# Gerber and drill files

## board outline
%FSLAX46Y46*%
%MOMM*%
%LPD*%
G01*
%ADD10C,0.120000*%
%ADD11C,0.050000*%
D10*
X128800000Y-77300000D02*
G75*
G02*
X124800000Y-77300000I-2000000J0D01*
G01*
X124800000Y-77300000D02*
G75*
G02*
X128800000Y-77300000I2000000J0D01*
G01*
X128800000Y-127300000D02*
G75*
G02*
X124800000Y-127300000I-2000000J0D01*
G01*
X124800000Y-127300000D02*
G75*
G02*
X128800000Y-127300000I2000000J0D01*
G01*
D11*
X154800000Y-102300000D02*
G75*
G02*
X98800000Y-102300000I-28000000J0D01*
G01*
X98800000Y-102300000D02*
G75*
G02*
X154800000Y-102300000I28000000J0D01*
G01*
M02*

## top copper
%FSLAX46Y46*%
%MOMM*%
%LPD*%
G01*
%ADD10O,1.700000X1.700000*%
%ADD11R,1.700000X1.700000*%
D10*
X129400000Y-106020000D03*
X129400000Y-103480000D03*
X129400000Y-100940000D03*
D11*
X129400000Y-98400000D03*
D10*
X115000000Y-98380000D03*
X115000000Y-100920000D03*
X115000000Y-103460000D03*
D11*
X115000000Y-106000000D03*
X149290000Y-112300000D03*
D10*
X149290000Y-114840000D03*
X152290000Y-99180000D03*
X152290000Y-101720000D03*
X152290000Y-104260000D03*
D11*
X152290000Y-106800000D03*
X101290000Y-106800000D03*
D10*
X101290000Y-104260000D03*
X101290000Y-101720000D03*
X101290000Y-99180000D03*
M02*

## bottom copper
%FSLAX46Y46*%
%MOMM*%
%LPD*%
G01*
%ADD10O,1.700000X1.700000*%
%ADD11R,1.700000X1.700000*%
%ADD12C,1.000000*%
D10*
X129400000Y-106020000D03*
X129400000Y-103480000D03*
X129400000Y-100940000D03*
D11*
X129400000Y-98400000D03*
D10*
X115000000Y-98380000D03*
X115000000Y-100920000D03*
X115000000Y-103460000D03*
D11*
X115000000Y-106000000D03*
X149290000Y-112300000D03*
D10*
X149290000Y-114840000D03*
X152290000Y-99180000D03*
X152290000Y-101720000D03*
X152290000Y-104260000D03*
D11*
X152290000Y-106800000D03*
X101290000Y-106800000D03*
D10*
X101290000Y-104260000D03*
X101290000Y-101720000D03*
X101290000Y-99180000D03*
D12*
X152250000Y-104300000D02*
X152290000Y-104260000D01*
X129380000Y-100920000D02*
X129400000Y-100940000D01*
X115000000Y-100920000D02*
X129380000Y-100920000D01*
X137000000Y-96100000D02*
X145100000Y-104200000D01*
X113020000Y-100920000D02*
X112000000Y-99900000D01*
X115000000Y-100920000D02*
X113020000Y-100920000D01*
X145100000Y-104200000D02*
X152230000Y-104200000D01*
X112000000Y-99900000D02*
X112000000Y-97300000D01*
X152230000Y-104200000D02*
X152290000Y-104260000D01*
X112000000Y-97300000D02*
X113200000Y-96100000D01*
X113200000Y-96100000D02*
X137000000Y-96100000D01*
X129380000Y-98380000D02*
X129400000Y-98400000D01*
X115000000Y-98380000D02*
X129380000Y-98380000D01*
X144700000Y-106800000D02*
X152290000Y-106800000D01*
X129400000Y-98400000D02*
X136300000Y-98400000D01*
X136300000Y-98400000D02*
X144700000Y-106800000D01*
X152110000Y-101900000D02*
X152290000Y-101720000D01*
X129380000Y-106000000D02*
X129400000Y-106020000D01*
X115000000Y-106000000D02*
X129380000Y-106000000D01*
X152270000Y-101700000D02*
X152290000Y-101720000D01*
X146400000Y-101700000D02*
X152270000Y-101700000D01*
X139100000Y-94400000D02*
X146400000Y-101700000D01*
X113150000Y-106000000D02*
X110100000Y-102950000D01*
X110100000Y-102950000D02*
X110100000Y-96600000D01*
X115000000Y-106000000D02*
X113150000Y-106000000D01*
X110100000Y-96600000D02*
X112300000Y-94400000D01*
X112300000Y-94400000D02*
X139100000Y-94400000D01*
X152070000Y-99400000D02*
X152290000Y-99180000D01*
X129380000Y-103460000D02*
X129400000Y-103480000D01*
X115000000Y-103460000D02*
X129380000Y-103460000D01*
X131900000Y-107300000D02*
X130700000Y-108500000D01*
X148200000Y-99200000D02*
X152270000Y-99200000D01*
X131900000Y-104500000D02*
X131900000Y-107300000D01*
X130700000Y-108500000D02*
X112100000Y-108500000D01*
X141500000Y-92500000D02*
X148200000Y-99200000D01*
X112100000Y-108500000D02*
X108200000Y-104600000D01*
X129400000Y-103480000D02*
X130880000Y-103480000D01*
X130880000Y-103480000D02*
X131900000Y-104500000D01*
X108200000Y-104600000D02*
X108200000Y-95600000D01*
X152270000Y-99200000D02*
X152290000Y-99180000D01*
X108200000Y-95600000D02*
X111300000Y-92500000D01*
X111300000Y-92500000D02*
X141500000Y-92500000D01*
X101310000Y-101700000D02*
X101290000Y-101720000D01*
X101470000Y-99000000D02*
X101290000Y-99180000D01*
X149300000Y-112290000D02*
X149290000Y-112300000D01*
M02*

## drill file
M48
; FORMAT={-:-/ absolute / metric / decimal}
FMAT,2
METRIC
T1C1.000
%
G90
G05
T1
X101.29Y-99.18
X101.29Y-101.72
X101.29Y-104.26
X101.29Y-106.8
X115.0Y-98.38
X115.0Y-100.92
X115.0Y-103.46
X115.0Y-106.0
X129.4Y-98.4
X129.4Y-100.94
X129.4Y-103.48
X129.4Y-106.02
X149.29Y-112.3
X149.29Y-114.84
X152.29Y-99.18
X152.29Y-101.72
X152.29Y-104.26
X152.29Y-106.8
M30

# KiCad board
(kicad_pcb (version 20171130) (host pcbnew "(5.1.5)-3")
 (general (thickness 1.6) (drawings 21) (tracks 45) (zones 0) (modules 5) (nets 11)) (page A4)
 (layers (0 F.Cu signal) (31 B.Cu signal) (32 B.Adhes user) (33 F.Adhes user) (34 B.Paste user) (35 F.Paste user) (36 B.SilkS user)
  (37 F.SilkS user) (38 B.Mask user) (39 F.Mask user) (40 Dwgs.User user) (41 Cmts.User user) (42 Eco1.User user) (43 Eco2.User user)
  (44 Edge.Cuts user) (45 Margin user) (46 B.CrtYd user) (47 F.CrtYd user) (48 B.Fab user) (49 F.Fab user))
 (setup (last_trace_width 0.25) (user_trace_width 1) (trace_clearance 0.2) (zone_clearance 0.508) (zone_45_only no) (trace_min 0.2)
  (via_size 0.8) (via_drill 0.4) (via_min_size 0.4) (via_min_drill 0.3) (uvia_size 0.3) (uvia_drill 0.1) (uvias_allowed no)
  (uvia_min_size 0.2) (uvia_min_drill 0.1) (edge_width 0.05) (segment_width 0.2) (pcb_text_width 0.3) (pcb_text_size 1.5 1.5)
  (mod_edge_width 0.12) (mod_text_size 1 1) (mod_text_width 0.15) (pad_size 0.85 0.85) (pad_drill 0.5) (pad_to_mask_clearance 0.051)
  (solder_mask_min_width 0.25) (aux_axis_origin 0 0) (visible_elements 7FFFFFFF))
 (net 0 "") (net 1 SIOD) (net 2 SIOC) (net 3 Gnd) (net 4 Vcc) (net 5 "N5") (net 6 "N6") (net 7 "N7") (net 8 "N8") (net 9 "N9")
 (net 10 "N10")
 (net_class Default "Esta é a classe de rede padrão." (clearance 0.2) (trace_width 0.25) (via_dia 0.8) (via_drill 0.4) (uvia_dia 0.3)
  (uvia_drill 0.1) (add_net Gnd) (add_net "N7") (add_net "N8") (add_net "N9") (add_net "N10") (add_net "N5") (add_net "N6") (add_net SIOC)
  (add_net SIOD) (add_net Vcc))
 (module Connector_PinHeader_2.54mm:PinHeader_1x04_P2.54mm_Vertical (layer F.Cu) (at 129.4 98.4)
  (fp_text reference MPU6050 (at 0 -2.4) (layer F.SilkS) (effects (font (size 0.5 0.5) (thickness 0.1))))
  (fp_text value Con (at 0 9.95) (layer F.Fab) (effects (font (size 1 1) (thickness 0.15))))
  (pad 4 thru_hole oval (at 0 7.62) (size 1.7 1.7) (drill 1) (layers *.Cu *.Mask) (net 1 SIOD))
  (pad 3 thru_hole oval (at 0 5.08) (size 1.7 1.7) (drill 1) (layers *.Cu *.Mask) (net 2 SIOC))
  (pad 2 thru_hole oval (at 0 2.54) (size 1.7 1.7) (drill 1) (layers *.Cu *.Mask) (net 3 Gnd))
  (pad 1 thru_hole rect (at 0 0) (size 1.7 1.7) (drill 1) (layers *.Cu *.Mask) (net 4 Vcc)))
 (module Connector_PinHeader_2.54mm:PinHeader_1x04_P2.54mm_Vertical (layer F.Cu) (at 115 106 180)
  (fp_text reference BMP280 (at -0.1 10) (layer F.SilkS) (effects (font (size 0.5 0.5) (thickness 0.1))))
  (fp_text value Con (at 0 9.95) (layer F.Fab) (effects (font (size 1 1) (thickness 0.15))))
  (pad 4 thru_hole oval (at 0 7.62 180) (size 1.7 1.7) (drill 1) (layers *.Cu *.Mask) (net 4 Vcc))
  (pad 3 thru_hole oval (at 0 5.08 180) (size 1.7 1.7) (drill 1) (layers *.Cu *.Mask) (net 3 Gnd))
  (pad 2 thru_hole oval (at 0 2.54 180) (size 1.7 1.7) (drill 1) (layers *.Cu *.Mask) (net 2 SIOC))
  (pad 1 thru_hole rect (at 0 0 180) (size 1.7 1.7) (drill 1) (layers *.Cu *.Mask) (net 1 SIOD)))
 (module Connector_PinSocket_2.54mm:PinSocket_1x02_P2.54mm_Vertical (layer F.Cu) (at 149.29 112.3)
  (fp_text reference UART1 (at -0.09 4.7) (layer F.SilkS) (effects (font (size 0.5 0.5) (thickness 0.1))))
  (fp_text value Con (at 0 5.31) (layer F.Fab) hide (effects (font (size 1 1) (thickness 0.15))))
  (pad 1 thru_hole rect (at 0 0) (size 1.7 1.7) (drill 1) (layers *.Cu *.Mask) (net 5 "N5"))
  (pad 2 thru_hole oval (at 0 2.54) (size 1.7 1.7) (drill 1) (layers *.Cu *.Mask) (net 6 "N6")))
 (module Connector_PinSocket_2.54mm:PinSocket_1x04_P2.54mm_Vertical (layer F.Cu) (at 152.29 106.8 180)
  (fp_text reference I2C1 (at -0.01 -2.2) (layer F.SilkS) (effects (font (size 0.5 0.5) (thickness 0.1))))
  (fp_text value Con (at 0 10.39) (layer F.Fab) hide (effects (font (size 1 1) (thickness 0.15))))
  (pad 4 thru_hole oval (at 0 7.62 180) (size 1.7 1.7) (drill 1) (layers *.Cu *.Mask) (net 2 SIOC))
  (pad 3 thru_hole oval (at 0 5.08 180) (size 1.7 1.7) (drill 1) (layers *.Cu *.Mask) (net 1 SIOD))
  (pad 2 thru_hole oval (at 0 2.54 180) (size 1.7 1.7) (drill 1) (layers *.Cu *.Mask) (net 3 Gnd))
  (pad 1 thru_hole rect (at 0 0 180) (size 1.7 1.7) (drill 1) (layers *.Cu *.Mask) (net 4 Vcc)))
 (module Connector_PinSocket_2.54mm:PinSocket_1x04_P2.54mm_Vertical (layer F.Cu) (at 101.29 106.8 180)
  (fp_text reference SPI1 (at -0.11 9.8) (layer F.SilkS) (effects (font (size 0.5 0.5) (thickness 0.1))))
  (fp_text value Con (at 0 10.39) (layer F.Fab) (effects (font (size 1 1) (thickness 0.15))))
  (pad 1 thru_hole rect (at 0 0 180) (size 1.7 1.7) (drill 1) (layers *.Cu *.Mask) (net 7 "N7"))
  (pad 2 thru_hole oval (at 0 2.54 180) (size 1.7 1.7) (drill 1) (layers *.Cu *.Mask) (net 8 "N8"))
  (pad 3 thru_hole oval (at 0 5.08 180) (size 1.7 1.7) (drill 1) (layers *.Cu *.Mask) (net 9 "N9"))
  (pad 4 thru_hole oval (at 0 7.62 180) (size 1.7 1.7) (drill 1) (layers *.Cu *.Mask) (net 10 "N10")))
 (gr_circle (center 126.8 77.3) (end 128.8 77.3) (layer Edge.Cuts) (width 0.12))
 (gr_circle (center 126.8 127.3) (end 128.8 127.3) (layer Edge.Cuts) (width 0.12))
 (gr_circle (center 126.8 102.3) (end 154.8 102.3) (layer Edge.Cuts) (width 0.05))
 (segment (start 152.25 104.3) (end 152.29 104.26) (width 1) (layer B.Cu) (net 3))
 (segment (start 129.38 100.92) (end 129.4 100.94) (width 1) (layer B.Cu) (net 3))
 (segment (start 115 100.92) (end 129.38 100.92) (width 1) (layer B.Cu) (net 3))
 (segment (start 137 96.1) (end 145.1 104.2) (width 1) (layer B.Cu) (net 3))
 (segment (start 113.02 100.92) (end 112 99.9) (width 1) (layer B.Cu) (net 3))
 (segment (start 115 100.92) (end 113.02 100.92) (width 1) (layer B.Cu) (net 3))
 (segment (start 145.1 104.2) (end 152.23 104.2) (width 1) (layer B.Cu) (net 3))
 (segment (start 112 99.9) (end 112 97.3) (width 1) (layer B.Cu) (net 3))
 (segment (start 152.23 104.2) (end 152.29 104.26) (width 1) (layer B.Cu) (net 3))
 (segment (start 112 97.3) (end 113.2 96.1) (width 1) (layer B.Cu) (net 3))
 (segment (start 113.2 96.1) (end 137 96.1) (width 1) (layer B.Cu) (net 3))
 (segment (start 129.38 98.38) (end 129.4 98.4) (width 1) (layer B.Cu) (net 4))
 (segment (start 115 98.38) (end 129.38 98.38) (width 1) (layer B.Cu) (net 4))
 (segment (start 144.7 106.8) (end 152.29 106.8) (width 1) (layer B.Cu) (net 4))
 (segment (start 129.4 98.4) (end 136.3 98.4) (width 1) (layer B.Cu) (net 4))
 (segment (start 136.3 98.4) (end 144.7 106.8) (width 1) (layer B.Cu) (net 4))
 (segment (start 152.11 101.9) (end 152.29 101.72) (width 1) (layer B.Cu) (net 1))
 (segment (start 129.38 106) (end 129.4 106.02) (width 1) (layer B.Cu) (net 1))
 (segment (start 115 106) (end 129.38 106) (width 1) (layer B.Cu) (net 1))
 (segment (start 152.27 101.7) (end 152.29 101.72) (width 1) (layer B.Cu) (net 1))
 (segment (start 146.4 101.7) (end 152.27 101.7) (width 1) (layer B.Cu) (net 1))
 (segment (start 139.1 94.4) (end 146.4 101.7) (width 1) (layer B.Cu) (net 1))
 (segment (start 113.15 106) (end 110.1 102.95) (width 1) (layer B.Cu) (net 1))
 (segment (start 110.1 102.95) (end 110.1 96.6) (width 1) (layer B.Cu) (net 1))
 (segment (start 115 106) (end 113.15 106) (width 1) (layer B.Cu) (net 1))
 (segment (start 110.1 96.6) (end 112.3 94.4) (width 1) (layer B.Cu) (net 1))
 (segment (start 112.3 94.4) (end 139.1 94.4) (width 1) (layer B.Cu) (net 1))
 (segment (start 152.07 99.4) (end 152.29 99.18) (width 1) (layer B.Cu) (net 2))
 (segment (start 129.38 103.46) (end 129.4 103.48) (width 1) (layer B.Cu) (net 2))
 (segment (start 115 103.46) (end 129.38 103.46) (width 1) (layer B.Cu) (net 2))
 (segment (start 131.9 107.3) (end 130.7 108.5) (width 1) (layer B.Cu) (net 2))
 (segment (start 148.2 99.2) (end 152.27 99.2) (width 1) (layer B.Cu) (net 2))
 (segment (start 131.9 104.5) (end 131.9 107.3) (width 1) (layer B.Cu) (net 2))
 (segment (start 130.7 108.5) (end 112.1 108.5) (width 1) (layer B.Cu) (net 2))
 (segment (start 141.5 92.5) (end 148.2 99.2) (width 1) (layer B.Cu) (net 2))
 (segment (start 112.1 108.5) (end 108.2 104.6) (width 1) (layer B.Cu) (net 2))
 (segment (start 129.4 103.48) (end 130.88 103.48) (width 1) (layer B.Cu) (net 2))
 (segment (start 130.88 103.48) (end 131.9 104.5) (width 1) (layer B.Cu) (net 2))
 (segment (start 108.2 104.6) (end 108.2 95.6) (width 1) (layer B.Cu) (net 2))
 (segment (start 152.27 99.2) (end 152.29 99.18) (width 1) (layer B.Cu) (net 2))
 (segment (start 108.2 95.6) (end 111.3 92.5) (width 1) (layer B.Cu) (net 2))
 (segment (start 111.3 92.5) (end 141.5 92.5) (width 1) (layer B.Cu) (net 2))
 (segment (start 101.31 101.7) (end 101.29 101.72) (width 1) (layer B.Cu) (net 9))
 (segment (start 101.47 99) (end 101.29 99.18) (width 1) (layer B.Cu) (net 10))
 (segment (start 149.3 112.29) (end 149.29 112.3) (width 1) (layer B.Cu) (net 5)))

